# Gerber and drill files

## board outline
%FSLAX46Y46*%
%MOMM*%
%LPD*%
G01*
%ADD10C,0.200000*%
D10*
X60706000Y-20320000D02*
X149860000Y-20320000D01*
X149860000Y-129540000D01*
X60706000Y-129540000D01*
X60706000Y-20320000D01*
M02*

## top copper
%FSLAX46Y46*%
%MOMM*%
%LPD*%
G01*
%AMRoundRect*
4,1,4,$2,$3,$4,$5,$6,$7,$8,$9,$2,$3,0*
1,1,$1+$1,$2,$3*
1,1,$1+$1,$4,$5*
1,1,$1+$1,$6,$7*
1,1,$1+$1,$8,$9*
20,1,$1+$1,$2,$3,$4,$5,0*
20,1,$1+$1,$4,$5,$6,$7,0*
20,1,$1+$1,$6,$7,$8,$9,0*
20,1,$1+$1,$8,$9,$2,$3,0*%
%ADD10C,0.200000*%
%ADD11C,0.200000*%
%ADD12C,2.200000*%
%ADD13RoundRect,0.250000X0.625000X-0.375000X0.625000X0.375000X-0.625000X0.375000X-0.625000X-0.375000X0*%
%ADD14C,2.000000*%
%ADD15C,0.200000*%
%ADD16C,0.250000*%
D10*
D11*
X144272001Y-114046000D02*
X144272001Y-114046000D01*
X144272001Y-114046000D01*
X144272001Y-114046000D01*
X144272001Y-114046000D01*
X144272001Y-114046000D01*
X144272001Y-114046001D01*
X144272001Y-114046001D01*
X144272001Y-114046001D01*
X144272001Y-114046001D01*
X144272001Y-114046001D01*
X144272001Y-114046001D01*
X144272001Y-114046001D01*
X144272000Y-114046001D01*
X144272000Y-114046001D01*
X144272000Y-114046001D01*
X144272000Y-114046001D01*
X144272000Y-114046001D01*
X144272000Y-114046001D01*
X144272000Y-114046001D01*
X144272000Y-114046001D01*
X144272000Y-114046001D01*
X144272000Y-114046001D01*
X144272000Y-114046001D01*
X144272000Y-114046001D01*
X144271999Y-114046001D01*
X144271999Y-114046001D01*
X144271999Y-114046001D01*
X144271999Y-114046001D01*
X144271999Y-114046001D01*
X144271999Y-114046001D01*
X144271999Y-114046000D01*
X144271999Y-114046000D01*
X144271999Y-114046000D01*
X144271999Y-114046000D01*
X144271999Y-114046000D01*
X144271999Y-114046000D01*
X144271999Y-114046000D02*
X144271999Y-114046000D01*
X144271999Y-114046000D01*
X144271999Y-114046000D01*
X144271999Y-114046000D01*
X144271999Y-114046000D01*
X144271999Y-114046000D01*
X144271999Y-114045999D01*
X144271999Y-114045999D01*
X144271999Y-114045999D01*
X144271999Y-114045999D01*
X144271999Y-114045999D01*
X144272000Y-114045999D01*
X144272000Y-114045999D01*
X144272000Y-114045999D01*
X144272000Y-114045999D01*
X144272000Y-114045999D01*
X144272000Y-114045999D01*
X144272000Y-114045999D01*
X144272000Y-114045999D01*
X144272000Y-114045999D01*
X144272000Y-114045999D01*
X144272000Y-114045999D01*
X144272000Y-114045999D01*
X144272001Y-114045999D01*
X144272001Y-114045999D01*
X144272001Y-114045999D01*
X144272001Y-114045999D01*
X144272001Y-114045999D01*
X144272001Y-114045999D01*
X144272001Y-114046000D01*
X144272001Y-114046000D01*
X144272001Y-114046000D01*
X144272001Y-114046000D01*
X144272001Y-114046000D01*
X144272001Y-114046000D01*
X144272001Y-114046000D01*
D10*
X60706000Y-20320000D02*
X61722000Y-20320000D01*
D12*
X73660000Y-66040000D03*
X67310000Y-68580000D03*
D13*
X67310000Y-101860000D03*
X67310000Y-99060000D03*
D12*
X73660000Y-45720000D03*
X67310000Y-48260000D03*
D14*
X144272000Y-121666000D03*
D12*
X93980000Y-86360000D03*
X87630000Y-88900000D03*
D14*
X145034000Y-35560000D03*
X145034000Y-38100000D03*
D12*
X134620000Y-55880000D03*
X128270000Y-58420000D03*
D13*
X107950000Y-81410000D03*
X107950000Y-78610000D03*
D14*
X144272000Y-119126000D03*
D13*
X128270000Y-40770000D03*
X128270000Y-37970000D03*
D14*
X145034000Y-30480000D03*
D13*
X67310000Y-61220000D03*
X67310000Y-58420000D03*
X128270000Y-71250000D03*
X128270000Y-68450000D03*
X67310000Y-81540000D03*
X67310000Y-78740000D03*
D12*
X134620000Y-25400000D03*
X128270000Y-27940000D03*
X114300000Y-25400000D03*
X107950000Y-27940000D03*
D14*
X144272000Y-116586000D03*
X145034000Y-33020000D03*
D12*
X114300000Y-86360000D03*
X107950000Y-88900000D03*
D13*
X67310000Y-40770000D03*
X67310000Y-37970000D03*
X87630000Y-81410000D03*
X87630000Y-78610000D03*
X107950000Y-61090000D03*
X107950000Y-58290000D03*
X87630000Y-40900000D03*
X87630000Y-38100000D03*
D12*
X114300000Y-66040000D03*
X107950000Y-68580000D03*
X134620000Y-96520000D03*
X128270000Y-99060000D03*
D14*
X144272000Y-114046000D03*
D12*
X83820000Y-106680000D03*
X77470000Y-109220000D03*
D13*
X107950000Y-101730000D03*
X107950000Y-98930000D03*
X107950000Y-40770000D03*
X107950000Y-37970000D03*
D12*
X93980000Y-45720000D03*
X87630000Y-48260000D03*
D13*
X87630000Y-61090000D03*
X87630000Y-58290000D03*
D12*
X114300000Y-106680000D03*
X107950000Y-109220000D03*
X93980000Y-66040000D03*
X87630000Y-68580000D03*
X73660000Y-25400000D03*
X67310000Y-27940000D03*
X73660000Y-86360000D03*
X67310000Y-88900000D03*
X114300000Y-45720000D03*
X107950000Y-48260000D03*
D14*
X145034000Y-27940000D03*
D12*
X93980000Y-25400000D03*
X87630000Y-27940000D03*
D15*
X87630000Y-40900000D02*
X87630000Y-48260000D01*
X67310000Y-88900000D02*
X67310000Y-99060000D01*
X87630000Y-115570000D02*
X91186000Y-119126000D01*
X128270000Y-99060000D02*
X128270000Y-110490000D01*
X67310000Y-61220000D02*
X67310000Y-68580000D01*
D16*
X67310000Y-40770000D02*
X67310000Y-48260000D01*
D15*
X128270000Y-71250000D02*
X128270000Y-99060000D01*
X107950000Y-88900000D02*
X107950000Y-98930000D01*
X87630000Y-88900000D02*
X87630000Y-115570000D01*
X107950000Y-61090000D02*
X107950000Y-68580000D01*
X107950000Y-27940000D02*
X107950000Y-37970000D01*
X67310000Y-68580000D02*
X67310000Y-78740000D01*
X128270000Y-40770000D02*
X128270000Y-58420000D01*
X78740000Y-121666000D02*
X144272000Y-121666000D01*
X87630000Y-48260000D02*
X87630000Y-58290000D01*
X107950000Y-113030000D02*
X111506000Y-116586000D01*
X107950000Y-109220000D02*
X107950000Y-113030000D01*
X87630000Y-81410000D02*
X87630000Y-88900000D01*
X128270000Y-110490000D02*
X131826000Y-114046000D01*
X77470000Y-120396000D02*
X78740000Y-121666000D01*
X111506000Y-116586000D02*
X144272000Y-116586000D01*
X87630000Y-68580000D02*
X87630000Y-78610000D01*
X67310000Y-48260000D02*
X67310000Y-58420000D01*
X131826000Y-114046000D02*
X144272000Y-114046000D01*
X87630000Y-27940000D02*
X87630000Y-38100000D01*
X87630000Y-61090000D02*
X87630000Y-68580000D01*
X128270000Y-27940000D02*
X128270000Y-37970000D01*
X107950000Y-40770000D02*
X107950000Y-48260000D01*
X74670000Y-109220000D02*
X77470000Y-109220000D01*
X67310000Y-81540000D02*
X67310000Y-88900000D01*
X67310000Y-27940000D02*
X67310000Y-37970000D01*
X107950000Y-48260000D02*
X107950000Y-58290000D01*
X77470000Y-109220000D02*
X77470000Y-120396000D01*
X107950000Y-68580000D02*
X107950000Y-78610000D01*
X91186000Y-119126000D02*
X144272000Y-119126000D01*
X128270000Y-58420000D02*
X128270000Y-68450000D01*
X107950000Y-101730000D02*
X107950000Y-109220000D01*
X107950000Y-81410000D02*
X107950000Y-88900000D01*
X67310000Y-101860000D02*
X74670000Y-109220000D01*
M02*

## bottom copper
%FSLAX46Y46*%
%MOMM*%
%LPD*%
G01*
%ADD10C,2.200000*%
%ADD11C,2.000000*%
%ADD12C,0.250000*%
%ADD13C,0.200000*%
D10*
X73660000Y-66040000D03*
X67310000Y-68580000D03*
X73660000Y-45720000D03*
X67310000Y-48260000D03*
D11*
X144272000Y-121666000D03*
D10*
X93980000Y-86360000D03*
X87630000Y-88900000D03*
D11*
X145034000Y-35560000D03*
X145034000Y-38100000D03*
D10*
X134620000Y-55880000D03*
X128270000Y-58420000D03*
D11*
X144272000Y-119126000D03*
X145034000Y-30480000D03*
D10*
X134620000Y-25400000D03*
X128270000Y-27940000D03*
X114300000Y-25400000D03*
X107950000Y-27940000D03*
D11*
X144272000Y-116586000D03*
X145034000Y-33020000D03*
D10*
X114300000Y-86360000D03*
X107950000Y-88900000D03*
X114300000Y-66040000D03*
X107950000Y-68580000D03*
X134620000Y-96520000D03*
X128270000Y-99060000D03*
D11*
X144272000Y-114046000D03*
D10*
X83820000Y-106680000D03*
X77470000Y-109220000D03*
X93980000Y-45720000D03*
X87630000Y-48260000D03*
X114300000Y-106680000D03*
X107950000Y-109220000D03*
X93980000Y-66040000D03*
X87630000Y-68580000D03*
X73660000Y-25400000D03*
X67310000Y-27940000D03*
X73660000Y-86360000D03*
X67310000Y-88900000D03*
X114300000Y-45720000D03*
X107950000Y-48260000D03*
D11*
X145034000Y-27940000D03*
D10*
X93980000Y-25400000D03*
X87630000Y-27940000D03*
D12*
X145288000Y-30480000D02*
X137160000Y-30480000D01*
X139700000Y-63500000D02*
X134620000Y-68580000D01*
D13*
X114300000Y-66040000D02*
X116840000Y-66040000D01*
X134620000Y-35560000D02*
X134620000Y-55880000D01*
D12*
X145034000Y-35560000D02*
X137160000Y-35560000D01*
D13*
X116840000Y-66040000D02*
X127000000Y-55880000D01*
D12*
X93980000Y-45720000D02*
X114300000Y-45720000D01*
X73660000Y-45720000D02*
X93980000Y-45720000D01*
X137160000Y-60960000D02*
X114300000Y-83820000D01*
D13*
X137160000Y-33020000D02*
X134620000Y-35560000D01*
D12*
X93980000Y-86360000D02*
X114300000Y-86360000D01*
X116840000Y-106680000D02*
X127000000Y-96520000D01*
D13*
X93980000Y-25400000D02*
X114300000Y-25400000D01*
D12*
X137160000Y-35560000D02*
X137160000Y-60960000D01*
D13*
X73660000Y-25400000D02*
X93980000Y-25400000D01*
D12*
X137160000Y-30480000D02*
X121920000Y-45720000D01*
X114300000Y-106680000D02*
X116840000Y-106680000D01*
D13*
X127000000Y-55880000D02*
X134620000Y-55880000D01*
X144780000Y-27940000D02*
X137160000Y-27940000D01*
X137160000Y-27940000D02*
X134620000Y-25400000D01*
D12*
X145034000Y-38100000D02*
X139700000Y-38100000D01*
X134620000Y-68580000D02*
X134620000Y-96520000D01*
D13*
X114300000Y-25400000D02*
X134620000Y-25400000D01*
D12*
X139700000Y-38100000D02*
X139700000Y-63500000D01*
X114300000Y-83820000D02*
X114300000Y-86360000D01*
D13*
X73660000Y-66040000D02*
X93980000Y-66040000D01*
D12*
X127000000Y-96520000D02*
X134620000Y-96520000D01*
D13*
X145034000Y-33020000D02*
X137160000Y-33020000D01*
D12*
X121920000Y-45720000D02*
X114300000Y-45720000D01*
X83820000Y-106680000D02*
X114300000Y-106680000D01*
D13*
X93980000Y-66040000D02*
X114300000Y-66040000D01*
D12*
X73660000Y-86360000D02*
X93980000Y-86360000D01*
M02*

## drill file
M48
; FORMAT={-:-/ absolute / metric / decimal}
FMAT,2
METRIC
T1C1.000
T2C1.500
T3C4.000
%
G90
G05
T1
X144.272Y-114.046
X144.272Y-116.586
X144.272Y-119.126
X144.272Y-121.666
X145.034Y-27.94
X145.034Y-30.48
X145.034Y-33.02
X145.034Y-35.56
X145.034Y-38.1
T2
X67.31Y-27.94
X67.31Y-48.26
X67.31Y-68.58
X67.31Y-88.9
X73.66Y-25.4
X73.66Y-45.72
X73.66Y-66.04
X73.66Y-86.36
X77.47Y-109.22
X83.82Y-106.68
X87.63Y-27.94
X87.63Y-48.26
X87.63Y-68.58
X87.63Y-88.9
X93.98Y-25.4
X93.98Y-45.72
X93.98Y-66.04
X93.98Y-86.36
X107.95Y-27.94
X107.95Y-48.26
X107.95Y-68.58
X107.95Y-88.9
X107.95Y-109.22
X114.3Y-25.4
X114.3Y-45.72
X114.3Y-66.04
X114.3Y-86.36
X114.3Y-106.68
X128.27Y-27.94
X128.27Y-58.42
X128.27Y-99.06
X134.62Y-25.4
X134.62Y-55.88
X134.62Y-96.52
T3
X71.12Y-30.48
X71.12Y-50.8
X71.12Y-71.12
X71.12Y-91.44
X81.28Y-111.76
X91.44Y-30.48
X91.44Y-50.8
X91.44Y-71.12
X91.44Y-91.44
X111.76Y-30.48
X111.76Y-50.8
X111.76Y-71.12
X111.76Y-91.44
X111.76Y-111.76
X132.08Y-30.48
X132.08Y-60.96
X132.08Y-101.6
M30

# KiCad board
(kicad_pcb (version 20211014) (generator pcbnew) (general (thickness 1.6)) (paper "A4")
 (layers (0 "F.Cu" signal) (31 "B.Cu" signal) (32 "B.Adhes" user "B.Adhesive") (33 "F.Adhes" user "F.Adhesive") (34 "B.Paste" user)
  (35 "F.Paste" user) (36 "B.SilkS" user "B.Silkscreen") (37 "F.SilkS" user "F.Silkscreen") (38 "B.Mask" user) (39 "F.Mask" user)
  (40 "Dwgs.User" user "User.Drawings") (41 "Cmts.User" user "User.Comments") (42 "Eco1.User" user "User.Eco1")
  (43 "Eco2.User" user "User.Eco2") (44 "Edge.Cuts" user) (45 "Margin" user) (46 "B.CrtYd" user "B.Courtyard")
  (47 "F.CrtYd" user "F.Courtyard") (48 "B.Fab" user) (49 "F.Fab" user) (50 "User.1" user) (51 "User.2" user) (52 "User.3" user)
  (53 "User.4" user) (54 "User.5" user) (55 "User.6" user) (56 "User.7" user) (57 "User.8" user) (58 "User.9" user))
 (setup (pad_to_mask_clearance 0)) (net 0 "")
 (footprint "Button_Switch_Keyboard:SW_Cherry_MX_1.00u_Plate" (layer "F.Cu") (at 73.66 66.04)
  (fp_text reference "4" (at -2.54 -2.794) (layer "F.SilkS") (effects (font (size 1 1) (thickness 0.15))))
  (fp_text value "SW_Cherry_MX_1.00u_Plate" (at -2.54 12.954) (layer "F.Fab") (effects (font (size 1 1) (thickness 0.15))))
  (pad "" np_thru_hole circle (at -2.54 5.08) (size 4 4) (drill 4) (layers *.Cu *.Mask))
  (pad "1" thru_hole circle (at 0 0) (size 2.2 2.2) (drill 1.5) (layers *.Cu *.Mask))
  (pad "2" thru_hole circle (at -6.35 2.54) (size 2.2 2.2) (drill 1.5) (layers *.Cu *.Mask)))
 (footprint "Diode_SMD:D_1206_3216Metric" (layer "F.Cu") (at 67.31 100.46 90)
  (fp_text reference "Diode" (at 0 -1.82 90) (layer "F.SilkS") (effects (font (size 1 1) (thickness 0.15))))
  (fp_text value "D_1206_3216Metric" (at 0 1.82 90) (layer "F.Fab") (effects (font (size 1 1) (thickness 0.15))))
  (pad "1" smd roundrect (at -1.4 0 90) (size 1.25 1.75) (layers "F.Cu" "F.Paste" "F.Mask") (roundrect_rratio 0.2))
  (pad "2" smd roundrect (at 1.4 0 90) (size 1.25 1.75) (layers "F.Cu" "F.Paste" "F.Mask") (roundrect_rratio 0.2)))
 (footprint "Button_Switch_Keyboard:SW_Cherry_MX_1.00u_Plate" (layer "F.Cu") (at 73.66 45.72)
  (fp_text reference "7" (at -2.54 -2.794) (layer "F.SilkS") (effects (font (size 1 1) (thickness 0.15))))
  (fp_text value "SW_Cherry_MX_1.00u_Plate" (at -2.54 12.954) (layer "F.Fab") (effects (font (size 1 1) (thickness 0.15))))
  (pad "" np_thru_hole circle (at -2.54 5.08) (size 4 4) (drill 4) (layers *.Cu *.Mask))
  (pad "1" thru_hole circle (at 0 0) (size 2.2 2.2) (drill 1.5) (layers *.Cu *.Mask))
  (pad "2" thru_hole circle (at -6.35 2.54) (size 2.2 2.2) (drill 1.5) (layers *.Cu *.Mask)))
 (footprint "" (layer "F.Cu") (at 144.272 121.666)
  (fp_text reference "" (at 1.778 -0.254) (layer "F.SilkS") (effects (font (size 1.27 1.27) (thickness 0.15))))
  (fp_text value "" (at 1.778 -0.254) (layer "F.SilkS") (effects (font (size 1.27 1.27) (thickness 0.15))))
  (pad "1" thru_hole circle (at 0 0) (size 2 2) (drill 1) (layers *.Cu *.Mask)))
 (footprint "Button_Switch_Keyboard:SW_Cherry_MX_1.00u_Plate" (layer "F.Cu") (at 93.98 86.36)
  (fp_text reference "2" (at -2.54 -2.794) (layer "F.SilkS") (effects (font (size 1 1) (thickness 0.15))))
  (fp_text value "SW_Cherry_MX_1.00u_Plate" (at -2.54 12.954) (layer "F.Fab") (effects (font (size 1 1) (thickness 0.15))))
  (pad "" np_thru_hole circle (at -2.54 5.08) (size 4 4) (drill 4) (layers *.Cu *.Mask))
  (pad "1" thru_hole circle (at 0 0) (size 2.2 2.2) (drill 1.5) (layers *.Cu *.Mask))
  (pad "2" thru_hole circle (at -6.35 2.54) (size 2.2 2.2) (drill 1.5) (layers *.Cu *.Mask)))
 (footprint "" (layer "F.Cu") (at 145.034 35.56)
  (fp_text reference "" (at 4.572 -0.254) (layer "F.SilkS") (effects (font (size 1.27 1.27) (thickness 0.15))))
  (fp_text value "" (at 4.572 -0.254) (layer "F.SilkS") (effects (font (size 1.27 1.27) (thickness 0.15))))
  (pad "1" thru_hole circle (at 0 0) (size 2 2) (drill 1) (layers *.Cu *.Mask)))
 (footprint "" (layer "F.Cu") (at 145.034 38.1)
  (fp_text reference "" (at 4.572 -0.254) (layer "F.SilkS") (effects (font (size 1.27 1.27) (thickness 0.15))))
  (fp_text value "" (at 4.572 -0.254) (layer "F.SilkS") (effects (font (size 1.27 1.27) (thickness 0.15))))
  (pad "1" thru_hole circle (at 0 0) (size 2 2) (drill 1) (layers *.Cu *.Mask)))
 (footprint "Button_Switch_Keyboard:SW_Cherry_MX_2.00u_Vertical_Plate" (layer "F.Cu") (at 134.62 55.88)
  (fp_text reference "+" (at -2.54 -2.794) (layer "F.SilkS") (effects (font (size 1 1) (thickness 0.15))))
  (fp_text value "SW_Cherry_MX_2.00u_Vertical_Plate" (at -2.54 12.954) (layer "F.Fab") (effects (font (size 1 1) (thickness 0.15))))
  (pad "" np_thru_hole circle (at -2.54 5.08) (size 4 4) (drill 4) (layers *.Cu *.Mask))
  (pad "1" thru_hole circle (at 0 0) (size 2.2 2.2) (drill 1.5) (layers *.Cu *.Mask))
  (pad "2" thru_hole circle (at -6.35 2.54) (size 2.2 2.2) (drill 1.5) (layers *.Cu *.Mask)))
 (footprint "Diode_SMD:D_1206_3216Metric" (layer "F.Cu") (at 107.95 80.01 90)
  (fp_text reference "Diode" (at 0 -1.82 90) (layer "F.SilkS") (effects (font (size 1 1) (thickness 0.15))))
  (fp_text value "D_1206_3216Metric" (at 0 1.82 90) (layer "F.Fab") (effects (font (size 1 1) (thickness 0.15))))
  (pad "1" smd roundrect (at -1.4 0 90) (size 1.25 1.75) (layers "F.Cu" "F.Paste" "F.Mask") (roundrect_rratio 0.2))
  (pad "2" smd roundrect (at 1.4 0 90) (size 1.25 1.75) (layers "F.Cu" "F.Paste" "F.Mask") (roundrect_rratio 0.2)))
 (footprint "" (layer "F.Cu") (at 144.272 119.126)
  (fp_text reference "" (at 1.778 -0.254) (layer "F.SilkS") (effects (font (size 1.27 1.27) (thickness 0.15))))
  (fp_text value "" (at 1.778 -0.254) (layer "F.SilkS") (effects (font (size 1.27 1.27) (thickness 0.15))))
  (pad "1" thru_hole circle (at 0 0) (size 2 2) (drill 1) (layers *.Cu *.Mask)))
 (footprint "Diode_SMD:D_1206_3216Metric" (layer "F.Cu") (at 128.27 39.37 90)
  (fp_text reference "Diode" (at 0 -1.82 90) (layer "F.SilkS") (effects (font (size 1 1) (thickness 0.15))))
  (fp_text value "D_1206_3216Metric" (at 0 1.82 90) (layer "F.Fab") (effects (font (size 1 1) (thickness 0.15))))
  (pad "1" smd roundrect (at -1.4 0 90) (size 1.25 1.75) (layers "F.Cu" "F.Paste" "F.Mask") (roundrect_rratio 0.2))
  (pad "2" smd roundrect (at 1.4 0 90) (size 1.25 1.75) (layers "F.Cu" "F.Paste" "F.Mask") (roundrect_rratio 0.2)))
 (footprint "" (layer "F.Cu") (at 145.034 30.48)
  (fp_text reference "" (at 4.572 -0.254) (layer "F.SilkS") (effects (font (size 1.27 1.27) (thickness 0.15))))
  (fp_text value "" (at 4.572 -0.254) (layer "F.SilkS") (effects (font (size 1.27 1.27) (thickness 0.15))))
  (pad "1" thru_hole circle (at 0 0) (size 2 2) (drill 1) (layers *.Cu *.Mask)))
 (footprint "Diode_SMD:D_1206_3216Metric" (layer "F.Cu") (at 67.31 59.82 90)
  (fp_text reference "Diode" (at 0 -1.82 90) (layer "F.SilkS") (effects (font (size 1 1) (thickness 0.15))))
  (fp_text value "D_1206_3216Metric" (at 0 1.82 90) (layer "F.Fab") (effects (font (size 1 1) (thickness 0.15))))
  (pad "1" smd roundrect (at -1.4 0 90) (size 1.25 1.75) (layers "F.Cu" "F.Paste" "F.Mask") (roundrect_rratio 0.2))
  (pad "2" smd roundrect (at 1.4 0 90) (size 1.25 1.75) (layers "F.Cu" "F.Paste" "F.Mask") (roundrect_rratio 0.2)))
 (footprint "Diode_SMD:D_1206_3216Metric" (layer "F.Cu") (at 128.27 69.85 90)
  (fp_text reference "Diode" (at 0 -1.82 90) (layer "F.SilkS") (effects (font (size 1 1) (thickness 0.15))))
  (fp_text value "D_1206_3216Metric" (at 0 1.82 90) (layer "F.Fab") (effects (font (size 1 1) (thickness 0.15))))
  (pad "1" smd roundrect (at -1.4 0 90) (size 1.25 1.75) (layers "F.Cu" "F.Paste" "F.Mask") (roundrect_rratio 0.2))
  (pad "2" smd roundrect (at 1.4 0 90) (size 1.25 1.75) (layers "F.Cu" "F.Paste" "F.Mask") (roundrect_rratio 0.2)))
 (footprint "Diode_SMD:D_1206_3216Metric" (layer "F.Cu") (at 67.31 80.14 90)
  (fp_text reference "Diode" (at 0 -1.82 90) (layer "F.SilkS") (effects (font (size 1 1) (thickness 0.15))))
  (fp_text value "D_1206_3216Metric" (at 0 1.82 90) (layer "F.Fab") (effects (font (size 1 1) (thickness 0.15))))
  (pad "1" smd roundrect (at -1.4 0 90) (size 1.25 1.75) (layers "F.Cu" "F.Paste" "F.Mask") (roundrect_rratio 0.2))
  (pad "2" smd roundrect (at 1.4 0 90) (size 1.25 1.75) (layers "F.Cu" "F.Paste" "F.Mask") (roundrect_rratio 0.2)))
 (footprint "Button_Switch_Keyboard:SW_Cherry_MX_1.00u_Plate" (layer "F.Cu") (at 134.62 25.4)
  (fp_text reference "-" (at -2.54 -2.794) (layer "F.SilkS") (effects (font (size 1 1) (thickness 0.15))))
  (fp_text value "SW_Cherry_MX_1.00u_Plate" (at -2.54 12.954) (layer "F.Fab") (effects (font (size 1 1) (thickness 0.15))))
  (pad "" np_thru_hole circle (at -2.54 5.08) (size 4 4) (drill 4) (layers *.Cu *.Mask))
  (pad "1" thru_hole circle (at 0 0) (size 2.2 2.2) (drill 1.5) (layers *.Cu *.Mask))
  (pad "2" thru_hole circle (at -6.35 2.54) (size 2.2 2.2) (drill 1.5) (layers *.Cu *.Mask)))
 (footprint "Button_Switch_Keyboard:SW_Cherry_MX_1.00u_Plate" (layer "F.Cu") (at 114.3 25.4)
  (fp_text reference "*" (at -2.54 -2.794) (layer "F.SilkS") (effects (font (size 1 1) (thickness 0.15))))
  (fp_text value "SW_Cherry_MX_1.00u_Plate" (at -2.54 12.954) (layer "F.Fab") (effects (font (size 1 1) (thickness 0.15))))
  (pad "" np_thru_hole circle (at -2.54 5.08) (size 4 4) (drill 4) (layers *.Cu *.Mask))
  (pad "1" thru_hole circle (at 0 0) (size 2.2 2.2) (drill 1.5) (layers *.Cu *.Mask))
  (pad "2" thru_hole circle (at -6.35 2.54) (size 2.2 2.2) (drill 1.5) (layers *.Cu *.Mask)))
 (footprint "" (layer "F.Cu") (at 144.272 116.586)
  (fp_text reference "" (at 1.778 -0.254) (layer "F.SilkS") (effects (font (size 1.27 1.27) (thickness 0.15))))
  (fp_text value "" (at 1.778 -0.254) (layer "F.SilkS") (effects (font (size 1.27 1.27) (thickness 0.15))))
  (pad "1" thru_hole circle (at 0 0) (size 2 2) (drill 1) (layers *.Cu *.Mask)))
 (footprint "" (layer "F.Cu") (at 145.034 33.02)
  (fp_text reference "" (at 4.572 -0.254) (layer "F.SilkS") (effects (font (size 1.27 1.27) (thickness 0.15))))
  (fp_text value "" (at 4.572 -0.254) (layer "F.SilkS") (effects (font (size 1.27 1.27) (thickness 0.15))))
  (pad "1" thru_hole circle (at 0 0) (size 2 2) (drill 1) (layers *.Cu *.Mask)))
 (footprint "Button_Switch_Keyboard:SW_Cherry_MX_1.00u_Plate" (layer "F.Cu") (at 114.3 86.36)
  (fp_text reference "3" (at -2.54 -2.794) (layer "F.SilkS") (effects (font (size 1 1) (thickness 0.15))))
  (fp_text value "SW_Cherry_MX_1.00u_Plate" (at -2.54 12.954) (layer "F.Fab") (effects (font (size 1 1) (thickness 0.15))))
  (pad "" np_thru_hole circle (at -2.54 5.08) (size 4 4) (drill 4) (layers *.Cu *.Mask))
  (pad "1" thru_hole circle (at 0 0) (size 2.2 2.2) (drill 1.5) (layers *.Cu *.Mask))
  (pad "2" thru_hole circle (at -6.35 2.54) (size 2.2 2.2) (drill 1.5) (layers *.Cu *.Mask)))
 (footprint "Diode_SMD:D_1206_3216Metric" (layer "F.Cu") (at 67.31 39.37 90)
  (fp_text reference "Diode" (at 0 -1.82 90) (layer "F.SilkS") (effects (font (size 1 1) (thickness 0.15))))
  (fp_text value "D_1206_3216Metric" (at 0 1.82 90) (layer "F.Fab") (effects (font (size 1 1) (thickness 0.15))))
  (pad "1" smd roundrect (at -1.4 0 90) (size 1.25 1.75) (layers "F.Cu" "F.Paste" "F.Mask") (roundrect_rratio 0.2))
  (pad "2" smd roundrect (at 1.4 0 90) (size 1.25 1.75) (layers "F.Cu" "F.Paste" "F.Mask") (roundrect_rratio 0.2)))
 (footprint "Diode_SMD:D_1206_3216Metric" (layer "F.Cu") (at 87.63 80.01 90)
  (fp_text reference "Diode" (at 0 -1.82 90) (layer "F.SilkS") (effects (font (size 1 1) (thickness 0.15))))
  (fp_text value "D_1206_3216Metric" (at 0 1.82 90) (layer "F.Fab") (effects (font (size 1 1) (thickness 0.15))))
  (pad "1" smd roundrect (at -1.4 0 90) (size 1.25 1.75) (layers "F.Cu" "F.Paste" "F.Mask") (roundrect_rratio 0.2))
  (pad "2" smd roundrect (at 1.4 0 90) (size 1.25 1.75) (layers "F.Cu" "F.Paste" "F.Mask") (roundrect_rratio 0.2)))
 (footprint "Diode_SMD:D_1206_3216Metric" (layer "F.Cu") (at 107.95 59.69 90)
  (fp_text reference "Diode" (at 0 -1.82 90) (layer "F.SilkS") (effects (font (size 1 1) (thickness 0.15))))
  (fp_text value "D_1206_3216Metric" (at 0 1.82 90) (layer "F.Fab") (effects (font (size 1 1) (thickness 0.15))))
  (pad "1" smd roundrect (at -1.4 0 90) (size 1.25 1.75) (layers "F.Cu" "F.Paste" "F.Mask") (roundrect_rratio 0.2))
  (pad "2" smd roundrect (at 1.4 0 90) (size 1.25 1.75) (layers "F.Cu" "F.Paste" "F.Mask") (roundrect_rratio 0.2)))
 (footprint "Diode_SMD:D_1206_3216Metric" (layer "F.Cu") (at 87.63 39.5 90)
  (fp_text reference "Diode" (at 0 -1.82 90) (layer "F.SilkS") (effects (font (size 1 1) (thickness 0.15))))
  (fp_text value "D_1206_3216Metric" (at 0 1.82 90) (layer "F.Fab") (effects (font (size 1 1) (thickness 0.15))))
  (pad "1" smd roundrect (at -1.4 0 90) (size 1.25 1.75) (layers "F.Cu" "F.Paste" "F.Mask") (roundrect_rratio 0.2))
  (pad "2" smd roundrect (at 1.4 0 90) (size 1.25 1.75) (layers "F.Cu" "F.Paste" "F.Mask") (roundrect_rratio 0.2)))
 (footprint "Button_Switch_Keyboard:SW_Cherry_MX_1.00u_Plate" (layer "F.Cu") (at 114.3 66.04)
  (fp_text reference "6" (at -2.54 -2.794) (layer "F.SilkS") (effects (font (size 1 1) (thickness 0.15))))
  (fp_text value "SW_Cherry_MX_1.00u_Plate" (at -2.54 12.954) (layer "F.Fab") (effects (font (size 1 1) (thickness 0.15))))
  (pad "" np_thru_hole circle (at -2.54 5.08) (size 4 4) (drill 4) (layers *.Cu *.Mask))
  (pad "1" thru_hole circle (at 0 0) (size 2.2 2.2) (drill 1.5) (layers *.Cu *.Mask))
  (pad "2" thru_hole circle (at -6.35 2.54) (size 2.2 2.2) (drill 1.5) (layers *.Cu *.Mask)))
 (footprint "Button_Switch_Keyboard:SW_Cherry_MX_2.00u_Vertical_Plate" (layer "F.Cu") (at 134.62 96.52)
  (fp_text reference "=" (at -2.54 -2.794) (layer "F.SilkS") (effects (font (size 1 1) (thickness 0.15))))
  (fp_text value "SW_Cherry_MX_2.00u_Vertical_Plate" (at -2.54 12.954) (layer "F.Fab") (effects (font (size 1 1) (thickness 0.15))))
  (pad "" np_thru_hole circle (at -2.54 5.08) (size 4 4) (drill 4) (layers *.Cu *.Mask))
  (pad "1" thru_hole circle (at 0 0) (size 2.2 2.2) (drill 1.5) (layers *.Cu *.Mask))
  (pad "2" thru_hole circle (at -6.35 2.54) (size 2.2 2.2) (drill 1.5) (layers *.Cu *.Mask)))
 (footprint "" (layer "F.Cu") (at 144.272 114.046)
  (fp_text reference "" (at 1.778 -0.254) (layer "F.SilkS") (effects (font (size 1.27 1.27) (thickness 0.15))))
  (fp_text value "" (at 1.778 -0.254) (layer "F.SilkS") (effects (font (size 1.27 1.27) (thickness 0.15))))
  (pad "1" thru_hole circle (at 0 0) (size 2 2) (drill 1) (layers *.Cu *.Mask)))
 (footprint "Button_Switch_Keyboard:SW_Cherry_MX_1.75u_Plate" (layer "F.Cu") (at 83.82 106.68)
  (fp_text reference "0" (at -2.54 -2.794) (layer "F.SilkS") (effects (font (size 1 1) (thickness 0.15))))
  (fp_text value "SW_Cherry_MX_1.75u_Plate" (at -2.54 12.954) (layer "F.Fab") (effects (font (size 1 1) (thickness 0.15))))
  (pad "" np_thru_hole circle (at -2.54 5.08) (size 4 4) (drill 4) (layers *.Cu *.Mask))
  (pad "1" thru_hole circle (at 0 0) (size 2.2 2.2) (drill 1.5) (layers *.Cu *.Mask))
  (pad "2" thru_hole circle (at -6.35 2.54) (size 2.2 2.2) (drill 1.5) (layers *.Cu *.Mask)))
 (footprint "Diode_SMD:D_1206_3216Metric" (layer "F.Cu") (at 107.95 100.33 90)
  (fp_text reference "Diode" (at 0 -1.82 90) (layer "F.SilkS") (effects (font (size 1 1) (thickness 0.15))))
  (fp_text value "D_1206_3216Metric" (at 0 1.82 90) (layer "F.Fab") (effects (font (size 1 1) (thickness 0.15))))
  (pad "1" smd roundrect (at -1.4 0 90) (size 1.25 1.75) (layers "F.Cu" "F.Paste" "F.Mask") (roundrect_rratio 0.2))
  (pad "2" smd roundrect (at 1.4 0 90) (size 1.25 1.75) (layers "F.Cu" "F.Paste" "F.Mask") (roundrect_rratio 0.2)))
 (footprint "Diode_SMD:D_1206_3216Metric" (layer "F.Cu") (at 107.95 39.37 90)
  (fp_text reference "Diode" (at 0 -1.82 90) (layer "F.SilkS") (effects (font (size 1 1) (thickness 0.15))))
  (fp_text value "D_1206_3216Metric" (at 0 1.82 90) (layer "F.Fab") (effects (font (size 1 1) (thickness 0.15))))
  (pad "1" smd roundrect (at -1.4 0 90) (size 1.25 1.75) (layers "F.Cu" "F.Paste" "F.Mask") (roundrect_rratio 0.2))
  (pad "2" smd roundrect (at 1.4 0 90) (size 1.25 1.75) (layers "F.Cu" "F.Paste" "F.Mask") (roundrect_rratio 0.2)))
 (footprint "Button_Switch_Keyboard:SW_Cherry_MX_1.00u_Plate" (layer "F.Cu") (at 93.98 45.72)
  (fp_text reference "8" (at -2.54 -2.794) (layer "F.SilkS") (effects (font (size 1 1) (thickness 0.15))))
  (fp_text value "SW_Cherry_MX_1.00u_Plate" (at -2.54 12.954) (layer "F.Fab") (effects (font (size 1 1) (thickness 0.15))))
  (pad "" np_thru_hole circle (at -2.54 5.08) (size 4 4) (drill 4) (layers *.Cu *.Mask))
  (pad "1" thru_hole circle (at 0 0) (size 2.2 2.2) (drill 1.5) (layers *.Cu *.Mask))
  (pad "2" thru_hole circle (at -6.35 2.54) (size 2.2 2.2) (drill 1.5) (layers *.Cu *.Mask)))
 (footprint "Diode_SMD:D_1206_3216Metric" (layer "F.Cu") (at 87.63 59.69 90)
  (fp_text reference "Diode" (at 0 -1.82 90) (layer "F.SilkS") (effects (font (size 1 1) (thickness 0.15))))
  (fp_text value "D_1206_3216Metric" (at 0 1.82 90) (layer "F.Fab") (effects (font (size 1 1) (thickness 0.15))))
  (pad "1" smd roundrect (at -1.4 0 90) (size 1.25 1.75) (layers "F.Cu" "F.Paste" "F.Mask") (roundrect_rratio 0.2))
  (pad "2" smd roundrect (at 1.4 0 90) (size 1.25 1.75) (layers "F.Cu" "F.Paste" "F.Mask") (roundrect_rratio 0.2)))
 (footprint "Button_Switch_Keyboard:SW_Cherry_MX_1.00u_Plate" (layer "F.Cu") (at 114.3 106.68)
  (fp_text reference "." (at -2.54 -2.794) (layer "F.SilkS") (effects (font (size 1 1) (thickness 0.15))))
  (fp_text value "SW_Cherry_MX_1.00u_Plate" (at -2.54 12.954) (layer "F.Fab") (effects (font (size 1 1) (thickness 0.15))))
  (pad "" np_thru_hole circle (at -2.54 5.08) (size 4 4) (drill 4) (layers *.Cu *.Mask))
  (pad "1" thru_hole circle (at 0 0) (size 2.2 2.2) (drill 1.5) (layers *.Cu *.Mask))
  (pad "2" thru_hole circle (at -6.35 2.54) (size 2.2 2.2) (drill 1.5) (layers *.Cu *.Mask)))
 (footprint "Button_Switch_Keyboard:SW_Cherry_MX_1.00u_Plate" (layer "F.Cu") (at 93.98 66.04)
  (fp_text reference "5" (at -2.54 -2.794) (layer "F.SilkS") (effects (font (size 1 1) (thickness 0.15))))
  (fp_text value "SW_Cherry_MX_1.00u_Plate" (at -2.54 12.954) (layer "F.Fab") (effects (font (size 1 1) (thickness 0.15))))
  (pad "" np_thru_hole circle (at -2.54 5.08) (size 4 4) (drill 4) (layers *.Cu *.Mask))
  (pad "1" thru_hole circle (at 0 0) (size 2.2 2.2) (drill 1.5) (layers *.Cu *.Mask))
  (pad "2" thru_hole circle (at -6.35 2.54) (size 2.2 2.2) (drill 1.5) (layers *.Cu *.Mask)))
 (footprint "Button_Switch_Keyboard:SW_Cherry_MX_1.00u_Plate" (layer "F.Cu") (at 73.66 25.4)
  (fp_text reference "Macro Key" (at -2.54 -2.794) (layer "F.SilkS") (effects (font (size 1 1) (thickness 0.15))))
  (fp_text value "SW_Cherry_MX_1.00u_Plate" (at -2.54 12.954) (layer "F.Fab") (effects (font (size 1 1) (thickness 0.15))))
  (pad "" np_thru_hole circle (at -2.54 5.08) (size 4 4) (drill 4) (layers *.Cu *.Mask))
  (pad "1" thru_hole circle (at 0 0) (size 2.2 2.2) (drill 1.5) (layers *.Cu *.Mask))
  (pad "2" thru_hole circle (at -6.35 2.54) (size 2.2 2.2) (drill 1.5) (layers *.Cu *.Mask)))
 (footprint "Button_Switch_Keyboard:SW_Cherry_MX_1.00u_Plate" (layer "F.Cu") (at 73.66 86.36)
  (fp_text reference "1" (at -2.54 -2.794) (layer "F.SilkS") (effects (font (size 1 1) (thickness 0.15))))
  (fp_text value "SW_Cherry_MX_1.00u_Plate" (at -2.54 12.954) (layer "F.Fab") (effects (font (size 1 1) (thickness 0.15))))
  (pad "" np_thru_hole circle (at -2.54 5.08) (size 4 4) (drill 4) (layers *.Cu *.Mask))
  (pad "1" thru_hole circle (at 0 0) (size 2.2 2.2) (drill 1.5) (layers *.Cu *.Mask))
  (pad "2" thru_hole circle (at -6.35 2.54) (size 2.2 2.2) (drill 1.5) (layers *.Cu *.Mask)))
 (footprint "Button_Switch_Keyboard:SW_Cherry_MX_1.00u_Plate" (layer "F.Cu") (at 114.3 45.72)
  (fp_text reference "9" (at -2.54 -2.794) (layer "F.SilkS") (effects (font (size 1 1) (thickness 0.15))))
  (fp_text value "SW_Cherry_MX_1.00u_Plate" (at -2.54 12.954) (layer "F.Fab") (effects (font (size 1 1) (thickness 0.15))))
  (pad "" np_thru_hole circle (at -2.54 5.08) (size 4 4) (drill 4) (layers *.Cu *.Mask))
  (pad "1" thru_hole circle (at 0 0) (size 2.2 2.2) (drill 1.5) (layers *.Cu *.Mask))
  (pad "2" thru_hole circle (at -6.35 2.54) (size 2.2 2.2) (drill 1.5) (layers *.Cu *.Mask)))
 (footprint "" (layer "F.Cu") (at 145.034 27.94)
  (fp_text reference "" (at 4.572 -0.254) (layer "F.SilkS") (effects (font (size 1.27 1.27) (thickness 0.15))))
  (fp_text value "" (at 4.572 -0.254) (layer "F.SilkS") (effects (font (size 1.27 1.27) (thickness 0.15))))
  (pad "1" thru_hole circle (at 0 0) (size 2 2) (drill 1) (layers *.Cu *.Mask)))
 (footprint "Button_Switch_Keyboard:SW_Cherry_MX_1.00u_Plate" (layer "F.Cu") (at 93.98 25.4)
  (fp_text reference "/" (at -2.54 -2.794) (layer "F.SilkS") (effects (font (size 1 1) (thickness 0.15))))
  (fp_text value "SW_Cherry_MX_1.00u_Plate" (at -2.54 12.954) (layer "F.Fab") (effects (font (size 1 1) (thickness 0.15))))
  (pad "" np_thru_hole circle (at -2.54 5.08) (size 4 4) (drill 4) (layers *.Cu *.Mask))
  (pad "1" thru_hole circle (at 0 0) (size 2.2 2.2) (drill 1.5) (layers *.Cu *.Mask))
  (pad "2" thru_hole circle (at -6.35 2.54) (size 2.2 2.2) (drill 1.5) (layers *.Cu *.Mask)))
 (gr_circle (center 144.272 114.046) (end 144.272 114.046) (layer "F.Cu") (width 0.2) (fill none))
 (gr_line (start 60.706 20.32) (end 61.722 20.32) (layer "F.Cu") (width 0.2))
 (gr_rect (start 149.86 20.32) (end 60.706 129.54) (layer "Edge.Cuts") (width 0.2) (fill none))
 (segment (start 87.63 40.9) (end 87.63 48.26) (width 0.2) (layer "F.Cu") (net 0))
 (segment (start 67.31 88.9) (end 67.31 99.06) (width 0.2) (layer "F.Cu") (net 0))
 (segment (start 87.63 115.57) (end 91.186 119.126) (width 0.2) (layer "F.Cu") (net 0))
 (segment (start 128.27 99.06) (end 128.27 110.49) (width 0.2) (layer "F.Cu") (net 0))
 (segment (start 67.31 61.22) (end 67.31 68.58) (width 0.2) (layer "F.Cu") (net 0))
 (segment (start 67.31 40.77) (end 67.31 48.26) (width 0.25) (layer "F.Cu") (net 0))
 (segment (start 128.27 71.25) (end 128.27 99.06) (width 0.2) (layer "F.Cu") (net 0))
 (segment (start 107.95 88.9) (end 107.95 98.93) (width 0.2) (layer "F.Cu") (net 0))
 (segment (start 87.63 88.9) (end 87.63 115.57) (width 0.2) (layer "F.Cu") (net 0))
 (segment (start 107.95 61.09) (end 107.95 68.58) (width 0.2) (layer "F.Cu") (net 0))
 (segment (start 107.95 27.94) (end 107.95 37.97) (width 0.2) (layer "F.Cu") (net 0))
 (segment (start 67.31 68.58) (end 67.31 78.74) (width 0.2) (layer "F.Cu") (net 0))
 (segment (start 128.27 40.77) (end 128.27 58.42) (width 0.2) (layer "F.Cu") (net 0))
 (segment (start 78.74 121.666) (end 144.272 121.666) (width 0.2) (layer "F.Cu") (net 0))
 (segment (start 87.63 48.26) (end 87.63 58.29) (width 0.2) (layer "F.Cu") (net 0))
 (segment (start 107.95 113.03) (end 111.506 116.586) (width 0.2) (layer "F.Cu") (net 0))
 (segment (start 107.95 109.22) (end 107.95 113.03) (width 0.2) (layer "F.Cu") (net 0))
 (segment (start 87.63 81.41) (end 87.63 88.9) (width 0.2) (layer "F.Cu") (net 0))
 (segment (start 128.27 110.49) (end 131.826 114.046) (width 0.2) (layer "F.Cu") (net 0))
 (segment (start 77.47 120.396) (end 78.74 121.666) (width 0.2) (layer "F.Cu") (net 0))
 (segment (start 111.506 116.586) (end 144.272 116.586) (width 0.2) (layer "F.Cu") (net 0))
 (segment (start 87.63 68.58) (end 87.63 78.61) (width 0.2) (layer "F.Cu") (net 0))
 (segment (start 67.31 48.26) (end 67.31 58.42) (width 0.2) (layer "F.Cu") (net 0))
 (segment (start 131.826 114.046) (end 144.272 114.046) (width 0.2) (layer "F.Cu") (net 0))
 (segment (start 87.63 27.94) (end 87.63 38.1) (width 0.2) (layer "F.Cu") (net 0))
 (segment (start 87.63 61.09) (end 87.63 68.58) (width 0.2) (layer "F.Cu") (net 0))
 (segment (start 128.27 27.94) (end 128.27 37.97) (width 0.2) (layer "F.Cu") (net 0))
 (segment (start 107.95 40.77) (end 107.95 48.26) (width 0.2) (layer "F.Cu") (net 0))
 (segment (start 74.67 109.22) (end 77.47 109.22) (width 0.2) (layer "F.Cu") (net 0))
 (segment (start 67.31 81.54) (end 67.31 88.9) (width 0.2) (layer "F.Cu") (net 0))
 (segment (start 67.31 27.94) (end 67.31 37.97) (width 0.2) (layer "F.Cu") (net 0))
 (segment (start 107.95 48.26) (end 107.95 58.29) (width 0.2) (layer "F.Cu") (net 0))
 (segment (start 77.47 109.22) (end 77.47 120.396) (width 0.2) (layer "F.Cu") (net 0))
 (segment (start 107.95 68.58) (end 107.95 78.61) (width 0.2) (layer "F.Cu") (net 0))
 (segment (start 91.186 119.126) (end 144.272 119.126) (width 0.2) (layer "F.Cu") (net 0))
 (segment (start 128.27 58.42) (end 128.27 68.45) (width 0.2) (layer "F.Cu") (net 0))
 (segment (start 107.95 101.73) (end 107.95 109.22) (width 0.2) (layer "F.Cu") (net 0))
 (segment (start 107.95 81.41) (end 107.95 88.9) (width 0.2) (layer "F.Cu") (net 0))
 (segment (start 67.31 101.86) (end 74.67 109.22) (width 0.2) (layer "F.Cu") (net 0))
 (segment (start 145.288 30.48) (end 137.16 30.48) (width 0.25) (layer "B.Cu") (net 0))
 (segment (start 139.7 63.5) (end 134.62 68.58) (width 0.25) (layer "B.Cu") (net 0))
 (segment (start 114.3 66.04) (end 116.84 66.04) (width 0.2) (layer "B.Cu") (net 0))
 (segment (start 134.62 35.56) (end 134.62 55.88) (width 0.2) (layer "B.Cu") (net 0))
 (segment (start 145.034 35.56) (end 137.16 35.56) (width 0.25) (layer "B.Cu") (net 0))
 (segment (start 116.84 66.04) (end 127 55.88) (width 0.2) (layer "B.Cu") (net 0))
 (segment (start 93.98 45.72) (end 114.3 45.72) (width 0.25) (layer "B.Cu") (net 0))
 (segment (start 73.66 45.72) (end 93.98 45.72) (width 0.25) (layer "B.Cu") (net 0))
 (segment (start 137.16 60.96) (end 114.3 83.82) (width 0.25) (layer "B.Cu") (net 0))
 (segment (start 137.16 33.02) (end 134.62 35.56) (width 0.2) (layer "B.Cu") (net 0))
 (segment (start 93.98 86.36) (end 114.3 86.36) (width 0.25) (layer "B.Cu") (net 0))
 (segment (start 116.84 106.68) (end 127 96.52) (width 0.25) (layer "B.Cu") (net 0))
 (segment (start 93.98 25.4) (end 114.3 25.4) (width 0.2) (layer "B.Cu") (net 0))
 (segment (start 137.16 35.56) (end 137.16 60.96) (width 0.25) (layer "B.Cu") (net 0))
 (segment (start 73.66 25.4) (end 93.98 25.4) (width 0.2) (layer "B.Cu") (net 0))
 (segment (start 137.16 30.48) (end 121.92 45.72) (width 0.25) (layer "B.Cu") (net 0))
 (segment (start 114.3 106.68) (end 116.84 106.68) (width 0.25) (layer "B.Cu") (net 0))
 (segment (start 127 55.88) (end 134.62 55.88) (width 0.2) (layer "B.Cu") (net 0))
 (segment (start 144.78 27.94) (end 137.16 27.94) (width 0.2) (layer "B.Cu") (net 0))
 (segment (start 137.16 27.94) (end 134.62 25.4) (width 0.2) (layer "B.Cu") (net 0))
 (segment (start 145.034 38.1) (end 139.7 38.1) (width 0.25) (layer "B.Cu") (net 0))
 (segment (start 134.62 68.58) (end 134.62 96.52) (width 0.25) (layer "B.Cu") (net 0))
 (segment (start 114.3 25.4) (end 134.62 25.4) (width 0.2) (layer "B.Cu") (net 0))
 (segment (start 139.7 38.1) (end 139.7 63.5) (width 0.25) (layer "B.Cu") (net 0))
 (segment (start 114.3 83.82) (end 114.3 86.36) (width 0.25) (layer "B.Cu") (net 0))
 (segment (start 73.66 66.04) (end 93.98 66.04) (width 0.2) (layer "B.Cu") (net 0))
 (segment (start 127 96.52) (end 134.62 96.52) (width 0.25) (layer "B.Cu") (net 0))
 (segment (start 145.034 33.02) (end 137.16 33.02) (width 0.2) (layer "B.Cu") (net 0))
 (segment (start 121.92 45.72) (end 114.3 45.72) (width 0.25) (layer "B.Cu") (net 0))
 (segment (start 83.82 106.68) (end 114.3 106.68) (width 0.25) (layer "B.Cu") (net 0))
 (segment (start 93.98 66.04) (end 114.3 66.04) (width 0.2) (layer "B.Cu") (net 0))
 (segment (start 73.66 86.36) (end 93.98 86.36) (width 0.25) (layer "B.Cu") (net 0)))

